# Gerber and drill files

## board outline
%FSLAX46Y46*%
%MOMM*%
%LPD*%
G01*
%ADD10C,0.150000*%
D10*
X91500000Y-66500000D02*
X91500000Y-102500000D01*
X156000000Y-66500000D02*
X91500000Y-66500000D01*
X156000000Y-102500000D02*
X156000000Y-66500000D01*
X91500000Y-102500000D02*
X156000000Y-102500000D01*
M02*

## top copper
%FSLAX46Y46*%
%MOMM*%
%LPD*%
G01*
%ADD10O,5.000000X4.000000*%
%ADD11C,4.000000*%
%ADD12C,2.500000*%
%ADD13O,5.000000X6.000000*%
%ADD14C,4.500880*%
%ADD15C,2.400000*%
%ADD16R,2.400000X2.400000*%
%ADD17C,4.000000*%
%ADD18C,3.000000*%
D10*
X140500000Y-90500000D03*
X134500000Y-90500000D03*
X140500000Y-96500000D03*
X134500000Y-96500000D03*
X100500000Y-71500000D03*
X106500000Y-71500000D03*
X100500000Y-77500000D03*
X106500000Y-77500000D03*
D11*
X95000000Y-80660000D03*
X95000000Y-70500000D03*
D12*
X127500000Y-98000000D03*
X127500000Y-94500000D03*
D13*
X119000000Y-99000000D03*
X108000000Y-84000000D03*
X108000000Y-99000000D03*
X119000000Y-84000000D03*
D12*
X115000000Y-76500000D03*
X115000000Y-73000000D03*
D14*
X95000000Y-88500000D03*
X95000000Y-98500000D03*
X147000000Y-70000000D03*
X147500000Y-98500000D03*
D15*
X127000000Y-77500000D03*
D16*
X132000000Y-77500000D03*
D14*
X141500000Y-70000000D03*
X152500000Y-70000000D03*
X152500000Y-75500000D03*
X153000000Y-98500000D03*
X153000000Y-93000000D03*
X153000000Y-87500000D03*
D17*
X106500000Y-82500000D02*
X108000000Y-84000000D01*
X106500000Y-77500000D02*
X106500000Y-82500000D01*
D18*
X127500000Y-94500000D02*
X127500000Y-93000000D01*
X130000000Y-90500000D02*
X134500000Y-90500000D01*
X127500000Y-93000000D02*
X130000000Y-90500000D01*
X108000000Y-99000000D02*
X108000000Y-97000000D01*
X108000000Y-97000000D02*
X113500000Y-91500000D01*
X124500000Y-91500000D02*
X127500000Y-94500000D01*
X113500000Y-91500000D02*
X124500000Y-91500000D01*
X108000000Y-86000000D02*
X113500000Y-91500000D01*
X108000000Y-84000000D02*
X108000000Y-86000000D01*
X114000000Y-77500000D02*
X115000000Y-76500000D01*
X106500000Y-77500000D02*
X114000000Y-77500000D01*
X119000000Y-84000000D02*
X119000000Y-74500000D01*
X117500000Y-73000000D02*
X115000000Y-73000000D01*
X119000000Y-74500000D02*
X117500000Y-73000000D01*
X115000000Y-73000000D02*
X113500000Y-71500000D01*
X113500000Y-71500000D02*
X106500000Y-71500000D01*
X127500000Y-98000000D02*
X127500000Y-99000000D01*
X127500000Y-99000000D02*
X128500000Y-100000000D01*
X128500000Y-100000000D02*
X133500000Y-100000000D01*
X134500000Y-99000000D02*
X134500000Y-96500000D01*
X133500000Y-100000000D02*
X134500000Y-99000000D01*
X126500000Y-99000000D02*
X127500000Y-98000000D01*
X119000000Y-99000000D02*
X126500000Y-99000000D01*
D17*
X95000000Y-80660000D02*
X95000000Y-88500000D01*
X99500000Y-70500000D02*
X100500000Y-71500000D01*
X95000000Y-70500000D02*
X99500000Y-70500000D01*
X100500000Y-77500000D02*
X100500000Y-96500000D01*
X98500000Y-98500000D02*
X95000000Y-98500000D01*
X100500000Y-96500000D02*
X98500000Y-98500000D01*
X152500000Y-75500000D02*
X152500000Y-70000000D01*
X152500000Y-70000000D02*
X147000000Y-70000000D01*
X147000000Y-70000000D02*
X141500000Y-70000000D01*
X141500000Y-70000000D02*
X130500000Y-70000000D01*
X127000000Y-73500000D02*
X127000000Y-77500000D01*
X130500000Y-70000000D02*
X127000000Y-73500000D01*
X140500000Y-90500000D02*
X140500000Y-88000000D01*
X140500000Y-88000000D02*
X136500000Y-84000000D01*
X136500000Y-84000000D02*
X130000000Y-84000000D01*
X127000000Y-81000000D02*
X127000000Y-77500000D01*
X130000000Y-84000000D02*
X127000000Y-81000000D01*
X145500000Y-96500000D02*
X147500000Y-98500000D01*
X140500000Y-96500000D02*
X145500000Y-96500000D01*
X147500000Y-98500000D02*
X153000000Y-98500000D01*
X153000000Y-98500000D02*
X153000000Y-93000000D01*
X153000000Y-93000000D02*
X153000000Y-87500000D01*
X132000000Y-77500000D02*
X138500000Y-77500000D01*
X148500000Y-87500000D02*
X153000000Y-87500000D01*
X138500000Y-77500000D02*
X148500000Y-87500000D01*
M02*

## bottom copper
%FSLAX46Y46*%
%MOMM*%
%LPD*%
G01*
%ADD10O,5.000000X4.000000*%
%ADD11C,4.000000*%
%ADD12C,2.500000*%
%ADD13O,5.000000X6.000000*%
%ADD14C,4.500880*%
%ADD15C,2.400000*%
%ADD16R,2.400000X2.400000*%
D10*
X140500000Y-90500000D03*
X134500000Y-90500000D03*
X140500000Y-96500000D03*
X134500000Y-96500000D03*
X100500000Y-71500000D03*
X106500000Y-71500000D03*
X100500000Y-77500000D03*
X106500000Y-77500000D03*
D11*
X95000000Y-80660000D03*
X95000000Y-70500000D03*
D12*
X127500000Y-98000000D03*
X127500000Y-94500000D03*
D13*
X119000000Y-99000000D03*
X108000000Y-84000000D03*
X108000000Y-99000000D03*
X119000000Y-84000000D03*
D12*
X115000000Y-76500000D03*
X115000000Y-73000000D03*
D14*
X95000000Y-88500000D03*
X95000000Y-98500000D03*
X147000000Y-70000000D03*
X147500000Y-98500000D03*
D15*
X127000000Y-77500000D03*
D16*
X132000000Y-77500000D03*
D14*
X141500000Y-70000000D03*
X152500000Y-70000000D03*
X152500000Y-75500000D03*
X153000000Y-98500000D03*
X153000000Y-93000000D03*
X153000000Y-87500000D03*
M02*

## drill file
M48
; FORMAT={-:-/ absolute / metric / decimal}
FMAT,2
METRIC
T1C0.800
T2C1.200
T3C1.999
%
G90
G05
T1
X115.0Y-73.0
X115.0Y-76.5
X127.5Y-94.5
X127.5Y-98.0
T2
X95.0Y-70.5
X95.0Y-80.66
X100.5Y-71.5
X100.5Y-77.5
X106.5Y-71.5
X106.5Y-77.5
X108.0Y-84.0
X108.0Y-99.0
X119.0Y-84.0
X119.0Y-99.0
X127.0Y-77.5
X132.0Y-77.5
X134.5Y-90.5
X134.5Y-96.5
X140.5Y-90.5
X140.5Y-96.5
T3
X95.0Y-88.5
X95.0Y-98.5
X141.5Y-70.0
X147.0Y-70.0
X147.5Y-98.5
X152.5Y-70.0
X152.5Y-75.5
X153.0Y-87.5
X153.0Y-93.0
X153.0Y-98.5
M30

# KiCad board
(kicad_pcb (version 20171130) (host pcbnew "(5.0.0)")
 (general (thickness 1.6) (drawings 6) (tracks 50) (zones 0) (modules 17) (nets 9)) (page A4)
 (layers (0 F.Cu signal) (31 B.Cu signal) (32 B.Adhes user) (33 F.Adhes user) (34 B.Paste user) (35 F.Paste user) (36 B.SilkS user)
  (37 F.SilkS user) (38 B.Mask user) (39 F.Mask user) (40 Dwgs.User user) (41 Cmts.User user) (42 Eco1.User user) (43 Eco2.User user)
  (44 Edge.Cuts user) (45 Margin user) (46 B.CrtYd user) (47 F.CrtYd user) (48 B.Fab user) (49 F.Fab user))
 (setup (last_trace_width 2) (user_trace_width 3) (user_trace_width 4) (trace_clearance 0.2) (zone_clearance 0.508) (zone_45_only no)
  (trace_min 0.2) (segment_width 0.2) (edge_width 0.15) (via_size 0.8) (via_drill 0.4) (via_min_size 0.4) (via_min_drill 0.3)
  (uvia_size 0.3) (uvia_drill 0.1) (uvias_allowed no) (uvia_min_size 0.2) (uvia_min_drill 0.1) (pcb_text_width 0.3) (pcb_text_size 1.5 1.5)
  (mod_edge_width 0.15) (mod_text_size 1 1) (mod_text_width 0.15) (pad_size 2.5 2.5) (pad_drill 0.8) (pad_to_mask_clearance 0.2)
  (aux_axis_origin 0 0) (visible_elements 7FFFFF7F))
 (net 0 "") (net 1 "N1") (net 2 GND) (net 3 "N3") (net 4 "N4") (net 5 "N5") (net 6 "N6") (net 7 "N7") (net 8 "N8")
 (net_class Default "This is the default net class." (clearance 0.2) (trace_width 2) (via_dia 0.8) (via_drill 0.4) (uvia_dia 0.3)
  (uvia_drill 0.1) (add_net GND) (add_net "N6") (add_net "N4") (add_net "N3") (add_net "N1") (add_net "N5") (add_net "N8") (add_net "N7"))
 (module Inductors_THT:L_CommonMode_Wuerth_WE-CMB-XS (layer F.Cu) (at 137.5 93.5)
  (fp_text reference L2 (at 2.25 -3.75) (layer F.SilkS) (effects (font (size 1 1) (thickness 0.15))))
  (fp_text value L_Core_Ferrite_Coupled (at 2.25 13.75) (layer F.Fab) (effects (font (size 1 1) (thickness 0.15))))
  (pad 2 thru_hole oval (at 3 -3) (size 5 4) (drill 1.2) (layers *.Cu *.Mask) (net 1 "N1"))
  (pad 1 thru_hole oval (at -3 -3) (size 5 4) (drill 1.2) (layers *.Cu *.Mask) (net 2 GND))
  (pad 4 thru_hole oval (at 3 3) (size 5 4) (drill 1.2) (layers *.Cu *.Mask) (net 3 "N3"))
  (pad 3 thru_hole oval (at -3 3) (size 5 4) (drill 1.2) (layers *.Cu *.Mask) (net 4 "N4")))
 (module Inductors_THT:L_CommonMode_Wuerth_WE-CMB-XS (layer F.Cu) (at 103.5 74.5)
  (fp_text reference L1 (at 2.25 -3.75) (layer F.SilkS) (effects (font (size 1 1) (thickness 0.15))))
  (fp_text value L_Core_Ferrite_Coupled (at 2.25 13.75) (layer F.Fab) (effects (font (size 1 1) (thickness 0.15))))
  (pad 1 thru_hole oval (at -3 -3) (size 5 4) (drill 1.2) (layers *.Cu *.Mask) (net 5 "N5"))
  (pad 2 thru_hole oval (at 3 -3) (size 5 4) (drill 1.2) (layers *.Cu *.Mask) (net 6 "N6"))
  (pad 3 thru_hole oval (at -3 3) (size 5 4) (drill 1.2) (layers *.Cu *.Mask) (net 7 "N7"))
  (pad 4 thru_hole oval (at 3 3) (size 5 4) (drill 1.2) (layers *.Cu *.Mask) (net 2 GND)))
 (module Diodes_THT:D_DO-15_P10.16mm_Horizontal (layer F.Cu) (at 95 70.5 270)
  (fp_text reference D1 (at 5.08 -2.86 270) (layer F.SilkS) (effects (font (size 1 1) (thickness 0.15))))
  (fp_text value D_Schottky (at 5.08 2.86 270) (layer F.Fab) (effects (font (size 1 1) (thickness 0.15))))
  (pad 2 thru_hole circle (at 10.16 0 270) (size 4 4) (drill 1.2) (layers *.Cu *.Mask) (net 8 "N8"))
  (pad 1 thru_hole circle (at 0 0 270) (size 4 4) (drill 1.2) (layers *.Cu *.Mask) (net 5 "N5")))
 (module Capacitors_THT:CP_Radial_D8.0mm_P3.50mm (layer F.Cu) (at 127.5 98 90)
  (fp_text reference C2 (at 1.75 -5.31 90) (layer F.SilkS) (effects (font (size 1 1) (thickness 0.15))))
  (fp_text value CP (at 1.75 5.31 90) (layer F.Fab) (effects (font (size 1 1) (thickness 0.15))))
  (pad 1 thru_hole circle (at 0 0 90) (size 2.5 2.5) (drill 0.8) (layers *.Cu *.Mask) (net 4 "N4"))
  (pad 2 thru_hole circle (at 3.5 0 90) (size 2.5 2.5) (drill 0.8) (layers *.Cu *.Mask) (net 2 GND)))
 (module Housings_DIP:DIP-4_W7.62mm (layer F.Cu) (at 113.5 91.5 270)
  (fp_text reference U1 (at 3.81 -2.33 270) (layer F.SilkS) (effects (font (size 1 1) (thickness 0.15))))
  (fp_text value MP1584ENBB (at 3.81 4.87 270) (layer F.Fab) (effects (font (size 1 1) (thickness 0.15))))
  (pad 4 thru_hole oval (at 7.5 -5.5 270) (size 6 5) (drill 1.2) (layers *.Cu *.Mask) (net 4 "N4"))
  (pad 2 thru_hole oval (at -7.5 5.5 270) (size 6 5) (drill 1.2) (layers *.Cu *.Mask) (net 2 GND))
  (pad 3 thru_hole oval (at 7.5 5.5 270) (size 6 5) (drill 1.2) (layers *.Cu *.Mask) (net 2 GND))
  (pad 1 thru_hole oval (at -7.5 -5.5 270) (size 6 5) (drill 1.2) (layers *.Cu *.Mask) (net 6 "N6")))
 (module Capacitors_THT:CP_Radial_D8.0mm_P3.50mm (layer F.Cu) (at 115 73 270)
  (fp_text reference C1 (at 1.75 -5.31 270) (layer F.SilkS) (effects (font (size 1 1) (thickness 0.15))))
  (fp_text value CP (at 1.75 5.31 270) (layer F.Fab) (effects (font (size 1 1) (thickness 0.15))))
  (pad 2 thru_hole circle (at 3.5 0 270) (size 2.5 2.5) (drill 0.8) (layers *.Cu *.Mask) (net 2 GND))
  (pad 1 thru_hole circle (at 0 0 270) (size 2.5 2.5) (drill 0.8) (layers *.Cu *.Mask) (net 6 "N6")))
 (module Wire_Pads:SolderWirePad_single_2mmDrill (layer F.Cu) (at 95 88.5)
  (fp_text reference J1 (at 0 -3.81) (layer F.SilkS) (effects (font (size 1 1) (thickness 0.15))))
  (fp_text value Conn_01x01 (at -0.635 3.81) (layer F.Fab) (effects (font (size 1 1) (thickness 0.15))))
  (pad 1 thru_hole circle (at 0 0) (size 4.50088 4.50088) (drill 1.99898) (layers *.Cu *.Mask) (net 8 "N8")))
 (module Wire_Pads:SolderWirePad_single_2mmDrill (layer F.Cu) (at 95 98.5)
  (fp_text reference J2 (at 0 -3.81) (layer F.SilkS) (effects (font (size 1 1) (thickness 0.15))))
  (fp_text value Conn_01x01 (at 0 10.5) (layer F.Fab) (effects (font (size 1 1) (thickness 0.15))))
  (pad 1 thru_hole circle (at 0 0) (size 4.50088 4.50088) (drill 1.99898) (layers *.Cu *.Mask) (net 7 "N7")))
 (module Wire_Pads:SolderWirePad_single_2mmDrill (layer F.Cu) (at 147 70)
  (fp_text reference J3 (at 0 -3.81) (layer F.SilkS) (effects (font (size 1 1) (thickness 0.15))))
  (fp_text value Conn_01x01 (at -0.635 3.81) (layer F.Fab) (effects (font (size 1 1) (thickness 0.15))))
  (pad 1 thru_hole circle (at 0 0) (size 4.50088 4.50088) (drill 1.99898) (layers *.Cu *.Mask) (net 1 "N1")))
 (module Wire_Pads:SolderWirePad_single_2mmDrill (layer F.Cu) (at 147.5 98.5)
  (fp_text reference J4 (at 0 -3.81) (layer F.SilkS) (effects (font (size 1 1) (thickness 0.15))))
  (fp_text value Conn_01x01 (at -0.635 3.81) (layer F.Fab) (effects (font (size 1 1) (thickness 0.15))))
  (pad 1 thru_hole circle (at 0 0) (size 4.50088 4.50088) (drill 1.99898) (layers *.Cu *.Mask) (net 3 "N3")))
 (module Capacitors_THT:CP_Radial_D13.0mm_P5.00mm (layer F.Cu) (at 132 77.5 180)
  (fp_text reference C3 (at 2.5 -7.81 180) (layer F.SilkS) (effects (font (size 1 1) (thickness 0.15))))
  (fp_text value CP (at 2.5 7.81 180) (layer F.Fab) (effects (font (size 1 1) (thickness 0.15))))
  (pad 2 thru_hole circle (at 5 0 180) (size 2.4 2.4) (drill 1.2) (layers *.Cu *.Mask) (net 1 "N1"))
  (pad 1 thru_hole rect (at 0 0 180) (size 2.4 2.4) (drill 1.2) (layers *.Cu *.Mask) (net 3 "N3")))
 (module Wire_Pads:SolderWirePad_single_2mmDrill (layer F.Cu) (at 141.5 70)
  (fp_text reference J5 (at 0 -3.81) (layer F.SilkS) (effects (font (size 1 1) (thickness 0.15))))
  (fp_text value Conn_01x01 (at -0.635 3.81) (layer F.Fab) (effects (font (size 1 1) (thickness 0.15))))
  (pad 1 thru_hole circle (at 0 0) (size 4.50088 4.50088) (drill 1.99898) (layers *.Cu *.Mask) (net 1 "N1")))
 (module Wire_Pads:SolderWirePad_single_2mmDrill (layer F.Cu) (at 152.5 70)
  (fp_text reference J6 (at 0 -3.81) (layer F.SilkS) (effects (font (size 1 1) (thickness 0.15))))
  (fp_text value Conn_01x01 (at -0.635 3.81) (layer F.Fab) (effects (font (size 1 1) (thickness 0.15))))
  (pad 1 thru_hole circle (at 0 0) (size 4.50088 4.50088) (drill 1.99898) (layers *.Cu *.Mask) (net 1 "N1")))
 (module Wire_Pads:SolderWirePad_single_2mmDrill (layer F.Cu) (at 152.5 75.5)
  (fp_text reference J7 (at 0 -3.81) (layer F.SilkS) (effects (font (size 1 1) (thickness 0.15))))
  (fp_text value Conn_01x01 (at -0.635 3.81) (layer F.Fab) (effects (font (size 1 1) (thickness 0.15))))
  (pad 1 thru_hole circle (at 0 0) (size 4.50088 4.50088) (drill 1.99898) (layers *.Cu *.Mask) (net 1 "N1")))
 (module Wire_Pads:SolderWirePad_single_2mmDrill (layer F.Cu) (at 153 98.5)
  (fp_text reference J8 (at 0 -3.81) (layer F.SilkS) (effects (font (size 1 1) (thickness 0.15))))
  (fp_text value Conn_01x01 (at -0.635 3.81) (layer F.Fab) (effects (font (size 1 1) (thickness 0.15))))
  (pad 1 thru_hole circle (at 0 0) (size 4.50088 4.50088) (drill 1.99898) (layers *.Cu *.Mask) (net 3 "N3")))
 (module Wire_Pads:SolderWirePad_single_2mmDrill (layer F.Cu) (at 153 93)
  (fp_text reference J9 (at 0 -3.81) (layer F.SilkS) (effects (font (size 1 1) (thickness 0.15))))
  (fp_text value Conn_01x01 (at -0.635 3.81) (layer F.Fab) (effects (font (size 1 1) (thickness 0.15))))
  (pad 1 thru_hole circle (at 0 0) (size 4.50088 4.50088) (drill 1.99898) (layers *.Cu *.Mask) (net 3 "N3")))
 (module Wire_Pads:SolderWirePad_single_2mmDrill (layer F.Cu) (at 153 87.5)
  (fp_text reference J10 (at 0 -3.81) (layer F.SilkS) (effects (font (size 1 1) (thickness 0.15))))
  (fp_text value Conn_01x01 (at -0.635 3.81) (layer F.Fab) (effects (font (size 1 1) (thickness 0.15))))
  (pad 1 thru_hole circle (at 0 0) (size 4.50088 4.50088) (drill 1.99898) (layers *.Cu *.Mask) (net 3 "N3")))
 (gr_line (start 91.5 66.5) (end 91.5 102.5) (layer Edge.Cuts) (width 0.15))
 (gr_line (start 156 66.5) (end 91.5 66.5) (layer Edge.Cuts) (width 0.15))
 (gr_line (start 156 102.5) (end 156 66.5) (layer Edge.Cuts) (width 0.15))
 (gr_line (start 91.5 102.5) (end 156 102.5) (layer Edge.Cuts) (width 0.15))
 (segment (start 106.5 82.5) (end 108 84) (width 4) (layer F.Cu) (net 2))
 (segment (start 106.5 77.5) (end 106.5 82.5) (width 4) (layer F.Cu) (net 2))
 (segment (start 127.5 94.5) (end 127.5 93) (width 3) (layer F.Cu) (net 2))
 (segment (start 130 90.5) (end 134.5 90.5) (width 3) (layer F.Cu) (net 2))
 (segment (start 127.5 93) (end 130 90.5) (width 3) (layer F.Cu) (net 2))
 (segment (start 108 99) (end 108 97) (width 3) (layer F.Cu) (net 2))
 (segment (start 108 97) (end 113.5 91.5) (width 3) (layer F.Cu) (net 2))
 (segment (start 124.5 91.5) (end 127.5 94.5) (width 3) (layer F.Cu) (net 2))
 (segment (start 113.5 91.5) (end 124.5 91.5) (width 3) (layer F.Cu) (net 2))
 (segment (start 108 86) (end 113.5 91.5) (width 3) (layer F.Cu) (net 2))
 (segment (start 108 84) (end 108 86) (width 3) (layer F.Cu) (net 2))
 (segment (start 114 77.5) (end 115 76.5) (width 3) (layer F.Cu) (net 2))
 (segment (start 106.5 77.5) (end 114 77.5) (width 3) (layer F.Cu) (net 2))
 (segment (start 119 84) (end 119 74.5) (width 3) (layer F.Cu) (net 6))
 (segment (start 117.5 73) (end 115 73) (width 3) (layer F.Cu) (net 6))
 (segment (start 119 74.5) (end 117.5 73) (width 3) (layer F.Cu) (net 6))
 (segment (start 115 73) (end 113.5 71.5) (width 3) (layer F.Cu) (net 6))
 (segment (start 113.5 71.5) (end 106.5 71.5) (width 3) (layer F.Cu) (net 6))
 (segment (start 127.5 98) (end 127.5 99) (width 3) (layer F.Cu) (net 4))
 (segment (start 127.5 99) (end 128.5 100) (width 3) (layer F.Cu) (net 4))
 (segment (start 128.5 100) (end 133.5 100) (width 3) (layer F.Cu) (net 4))
 (segment (start 134.5 99) (end 134.5 96.5) (width 3) (layer F.Cu) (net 4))
 (segment (start 133.5 100) (end 134.5 99) (width 3) (layer F.Cu) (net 4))
 (segment (start 126.5 99) (end 127.5 98) (width 3) (layer F.Cu) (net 4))
 (segment (start 119 99) (end 126.5 99) (width 3) (layer F.Cu) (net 4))
 (segment (start 95 80.66) (end 95 88.5) (width 4) (layer F.Cu) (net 8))
 (segment (start 99.5 70.5) (end 100.5 71.5) (width 4) (layer F.Cu) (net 5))
 (segment (start 95 70.5) (end 99.5 70.5) (width 4) (layer F.Cu) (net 5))
 (segment (start 100.5 77.5) (end 100.5 96.5) (width 4) (layer F.Cu) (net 7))
 (segment (start 98.5 98.5) (end 95 98.5) (width 4) (layer F.Cu) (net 7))
 (segment (start 100.5 96.5) (end 98.5 98.5) (width 4) (layer F.Cu) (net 7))
 (segment (start 152.5 75.5) (end 152.5 70) (width 4) (layer F.Cu) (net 1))
 (segment (start 152.5 70) (end 147 70) (width 4) (layer F.Cu) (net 1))
 (segment (start 147 70) (end 141.5 70) (width 4) (layer F.Cu) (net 1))
 (segment (start 141.5 70) (end 130.5 70) (width 4) (layer F.Cu) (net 1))
 (segment (start 127 73.5) (end 127 77.5) (width 4) (layer F.Cu) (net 1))
 (segment (start 130.5 70) (end 127 73.5) (width 4) (layer F.Cu) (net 1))
 (segment (start 140.5 90.5) (end 140.5 88) (width 4) (layer F.Cu) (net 1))
 (segment (start 140.5 88) (end 136.5 84) (width 4) (layer F.Cu) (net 1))
 (segment (start 136.5 84) (end 130 84) (width 4) (layer F.Cu) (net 1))
 (segment (start 127 81) (end 127 77.5) (width 4) (layer F.Cu) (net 1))
 (segment (start 130 84) (end 127 81) (width 4) (layer F.Cu) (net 1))
 (segment (start 145.5 96.5) (end 147.5 98.5) (width 4) (layer F.Cu) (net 3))
 (segment (start 140.5 96.5) (end 145.5 96.5) (width 4) (layer F.Cu) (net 3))
 (segment (start 147.5 98.5) (end 153 98.5) (width 4) (layer F.Cu) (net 3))
 (segment (start 153 98.5) (end 153 93) (width 4) (layer F.Cu) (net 3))
 (segment (start 153 93) (end 153 87.5) (width 4) (layer F.Cu) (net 3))
 (segment (start 132 77.5) (end 138.5 77.5) (width 4) (layer F.Cu) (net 3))
 (segment (start 148.5 87.5) (end 153 87.5) (width 4) (layer F.Cu) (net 3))
 (segment (start 138.5 77.5) (end 148.5 87.5) (width 4) (layer F.Cu) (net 3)))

